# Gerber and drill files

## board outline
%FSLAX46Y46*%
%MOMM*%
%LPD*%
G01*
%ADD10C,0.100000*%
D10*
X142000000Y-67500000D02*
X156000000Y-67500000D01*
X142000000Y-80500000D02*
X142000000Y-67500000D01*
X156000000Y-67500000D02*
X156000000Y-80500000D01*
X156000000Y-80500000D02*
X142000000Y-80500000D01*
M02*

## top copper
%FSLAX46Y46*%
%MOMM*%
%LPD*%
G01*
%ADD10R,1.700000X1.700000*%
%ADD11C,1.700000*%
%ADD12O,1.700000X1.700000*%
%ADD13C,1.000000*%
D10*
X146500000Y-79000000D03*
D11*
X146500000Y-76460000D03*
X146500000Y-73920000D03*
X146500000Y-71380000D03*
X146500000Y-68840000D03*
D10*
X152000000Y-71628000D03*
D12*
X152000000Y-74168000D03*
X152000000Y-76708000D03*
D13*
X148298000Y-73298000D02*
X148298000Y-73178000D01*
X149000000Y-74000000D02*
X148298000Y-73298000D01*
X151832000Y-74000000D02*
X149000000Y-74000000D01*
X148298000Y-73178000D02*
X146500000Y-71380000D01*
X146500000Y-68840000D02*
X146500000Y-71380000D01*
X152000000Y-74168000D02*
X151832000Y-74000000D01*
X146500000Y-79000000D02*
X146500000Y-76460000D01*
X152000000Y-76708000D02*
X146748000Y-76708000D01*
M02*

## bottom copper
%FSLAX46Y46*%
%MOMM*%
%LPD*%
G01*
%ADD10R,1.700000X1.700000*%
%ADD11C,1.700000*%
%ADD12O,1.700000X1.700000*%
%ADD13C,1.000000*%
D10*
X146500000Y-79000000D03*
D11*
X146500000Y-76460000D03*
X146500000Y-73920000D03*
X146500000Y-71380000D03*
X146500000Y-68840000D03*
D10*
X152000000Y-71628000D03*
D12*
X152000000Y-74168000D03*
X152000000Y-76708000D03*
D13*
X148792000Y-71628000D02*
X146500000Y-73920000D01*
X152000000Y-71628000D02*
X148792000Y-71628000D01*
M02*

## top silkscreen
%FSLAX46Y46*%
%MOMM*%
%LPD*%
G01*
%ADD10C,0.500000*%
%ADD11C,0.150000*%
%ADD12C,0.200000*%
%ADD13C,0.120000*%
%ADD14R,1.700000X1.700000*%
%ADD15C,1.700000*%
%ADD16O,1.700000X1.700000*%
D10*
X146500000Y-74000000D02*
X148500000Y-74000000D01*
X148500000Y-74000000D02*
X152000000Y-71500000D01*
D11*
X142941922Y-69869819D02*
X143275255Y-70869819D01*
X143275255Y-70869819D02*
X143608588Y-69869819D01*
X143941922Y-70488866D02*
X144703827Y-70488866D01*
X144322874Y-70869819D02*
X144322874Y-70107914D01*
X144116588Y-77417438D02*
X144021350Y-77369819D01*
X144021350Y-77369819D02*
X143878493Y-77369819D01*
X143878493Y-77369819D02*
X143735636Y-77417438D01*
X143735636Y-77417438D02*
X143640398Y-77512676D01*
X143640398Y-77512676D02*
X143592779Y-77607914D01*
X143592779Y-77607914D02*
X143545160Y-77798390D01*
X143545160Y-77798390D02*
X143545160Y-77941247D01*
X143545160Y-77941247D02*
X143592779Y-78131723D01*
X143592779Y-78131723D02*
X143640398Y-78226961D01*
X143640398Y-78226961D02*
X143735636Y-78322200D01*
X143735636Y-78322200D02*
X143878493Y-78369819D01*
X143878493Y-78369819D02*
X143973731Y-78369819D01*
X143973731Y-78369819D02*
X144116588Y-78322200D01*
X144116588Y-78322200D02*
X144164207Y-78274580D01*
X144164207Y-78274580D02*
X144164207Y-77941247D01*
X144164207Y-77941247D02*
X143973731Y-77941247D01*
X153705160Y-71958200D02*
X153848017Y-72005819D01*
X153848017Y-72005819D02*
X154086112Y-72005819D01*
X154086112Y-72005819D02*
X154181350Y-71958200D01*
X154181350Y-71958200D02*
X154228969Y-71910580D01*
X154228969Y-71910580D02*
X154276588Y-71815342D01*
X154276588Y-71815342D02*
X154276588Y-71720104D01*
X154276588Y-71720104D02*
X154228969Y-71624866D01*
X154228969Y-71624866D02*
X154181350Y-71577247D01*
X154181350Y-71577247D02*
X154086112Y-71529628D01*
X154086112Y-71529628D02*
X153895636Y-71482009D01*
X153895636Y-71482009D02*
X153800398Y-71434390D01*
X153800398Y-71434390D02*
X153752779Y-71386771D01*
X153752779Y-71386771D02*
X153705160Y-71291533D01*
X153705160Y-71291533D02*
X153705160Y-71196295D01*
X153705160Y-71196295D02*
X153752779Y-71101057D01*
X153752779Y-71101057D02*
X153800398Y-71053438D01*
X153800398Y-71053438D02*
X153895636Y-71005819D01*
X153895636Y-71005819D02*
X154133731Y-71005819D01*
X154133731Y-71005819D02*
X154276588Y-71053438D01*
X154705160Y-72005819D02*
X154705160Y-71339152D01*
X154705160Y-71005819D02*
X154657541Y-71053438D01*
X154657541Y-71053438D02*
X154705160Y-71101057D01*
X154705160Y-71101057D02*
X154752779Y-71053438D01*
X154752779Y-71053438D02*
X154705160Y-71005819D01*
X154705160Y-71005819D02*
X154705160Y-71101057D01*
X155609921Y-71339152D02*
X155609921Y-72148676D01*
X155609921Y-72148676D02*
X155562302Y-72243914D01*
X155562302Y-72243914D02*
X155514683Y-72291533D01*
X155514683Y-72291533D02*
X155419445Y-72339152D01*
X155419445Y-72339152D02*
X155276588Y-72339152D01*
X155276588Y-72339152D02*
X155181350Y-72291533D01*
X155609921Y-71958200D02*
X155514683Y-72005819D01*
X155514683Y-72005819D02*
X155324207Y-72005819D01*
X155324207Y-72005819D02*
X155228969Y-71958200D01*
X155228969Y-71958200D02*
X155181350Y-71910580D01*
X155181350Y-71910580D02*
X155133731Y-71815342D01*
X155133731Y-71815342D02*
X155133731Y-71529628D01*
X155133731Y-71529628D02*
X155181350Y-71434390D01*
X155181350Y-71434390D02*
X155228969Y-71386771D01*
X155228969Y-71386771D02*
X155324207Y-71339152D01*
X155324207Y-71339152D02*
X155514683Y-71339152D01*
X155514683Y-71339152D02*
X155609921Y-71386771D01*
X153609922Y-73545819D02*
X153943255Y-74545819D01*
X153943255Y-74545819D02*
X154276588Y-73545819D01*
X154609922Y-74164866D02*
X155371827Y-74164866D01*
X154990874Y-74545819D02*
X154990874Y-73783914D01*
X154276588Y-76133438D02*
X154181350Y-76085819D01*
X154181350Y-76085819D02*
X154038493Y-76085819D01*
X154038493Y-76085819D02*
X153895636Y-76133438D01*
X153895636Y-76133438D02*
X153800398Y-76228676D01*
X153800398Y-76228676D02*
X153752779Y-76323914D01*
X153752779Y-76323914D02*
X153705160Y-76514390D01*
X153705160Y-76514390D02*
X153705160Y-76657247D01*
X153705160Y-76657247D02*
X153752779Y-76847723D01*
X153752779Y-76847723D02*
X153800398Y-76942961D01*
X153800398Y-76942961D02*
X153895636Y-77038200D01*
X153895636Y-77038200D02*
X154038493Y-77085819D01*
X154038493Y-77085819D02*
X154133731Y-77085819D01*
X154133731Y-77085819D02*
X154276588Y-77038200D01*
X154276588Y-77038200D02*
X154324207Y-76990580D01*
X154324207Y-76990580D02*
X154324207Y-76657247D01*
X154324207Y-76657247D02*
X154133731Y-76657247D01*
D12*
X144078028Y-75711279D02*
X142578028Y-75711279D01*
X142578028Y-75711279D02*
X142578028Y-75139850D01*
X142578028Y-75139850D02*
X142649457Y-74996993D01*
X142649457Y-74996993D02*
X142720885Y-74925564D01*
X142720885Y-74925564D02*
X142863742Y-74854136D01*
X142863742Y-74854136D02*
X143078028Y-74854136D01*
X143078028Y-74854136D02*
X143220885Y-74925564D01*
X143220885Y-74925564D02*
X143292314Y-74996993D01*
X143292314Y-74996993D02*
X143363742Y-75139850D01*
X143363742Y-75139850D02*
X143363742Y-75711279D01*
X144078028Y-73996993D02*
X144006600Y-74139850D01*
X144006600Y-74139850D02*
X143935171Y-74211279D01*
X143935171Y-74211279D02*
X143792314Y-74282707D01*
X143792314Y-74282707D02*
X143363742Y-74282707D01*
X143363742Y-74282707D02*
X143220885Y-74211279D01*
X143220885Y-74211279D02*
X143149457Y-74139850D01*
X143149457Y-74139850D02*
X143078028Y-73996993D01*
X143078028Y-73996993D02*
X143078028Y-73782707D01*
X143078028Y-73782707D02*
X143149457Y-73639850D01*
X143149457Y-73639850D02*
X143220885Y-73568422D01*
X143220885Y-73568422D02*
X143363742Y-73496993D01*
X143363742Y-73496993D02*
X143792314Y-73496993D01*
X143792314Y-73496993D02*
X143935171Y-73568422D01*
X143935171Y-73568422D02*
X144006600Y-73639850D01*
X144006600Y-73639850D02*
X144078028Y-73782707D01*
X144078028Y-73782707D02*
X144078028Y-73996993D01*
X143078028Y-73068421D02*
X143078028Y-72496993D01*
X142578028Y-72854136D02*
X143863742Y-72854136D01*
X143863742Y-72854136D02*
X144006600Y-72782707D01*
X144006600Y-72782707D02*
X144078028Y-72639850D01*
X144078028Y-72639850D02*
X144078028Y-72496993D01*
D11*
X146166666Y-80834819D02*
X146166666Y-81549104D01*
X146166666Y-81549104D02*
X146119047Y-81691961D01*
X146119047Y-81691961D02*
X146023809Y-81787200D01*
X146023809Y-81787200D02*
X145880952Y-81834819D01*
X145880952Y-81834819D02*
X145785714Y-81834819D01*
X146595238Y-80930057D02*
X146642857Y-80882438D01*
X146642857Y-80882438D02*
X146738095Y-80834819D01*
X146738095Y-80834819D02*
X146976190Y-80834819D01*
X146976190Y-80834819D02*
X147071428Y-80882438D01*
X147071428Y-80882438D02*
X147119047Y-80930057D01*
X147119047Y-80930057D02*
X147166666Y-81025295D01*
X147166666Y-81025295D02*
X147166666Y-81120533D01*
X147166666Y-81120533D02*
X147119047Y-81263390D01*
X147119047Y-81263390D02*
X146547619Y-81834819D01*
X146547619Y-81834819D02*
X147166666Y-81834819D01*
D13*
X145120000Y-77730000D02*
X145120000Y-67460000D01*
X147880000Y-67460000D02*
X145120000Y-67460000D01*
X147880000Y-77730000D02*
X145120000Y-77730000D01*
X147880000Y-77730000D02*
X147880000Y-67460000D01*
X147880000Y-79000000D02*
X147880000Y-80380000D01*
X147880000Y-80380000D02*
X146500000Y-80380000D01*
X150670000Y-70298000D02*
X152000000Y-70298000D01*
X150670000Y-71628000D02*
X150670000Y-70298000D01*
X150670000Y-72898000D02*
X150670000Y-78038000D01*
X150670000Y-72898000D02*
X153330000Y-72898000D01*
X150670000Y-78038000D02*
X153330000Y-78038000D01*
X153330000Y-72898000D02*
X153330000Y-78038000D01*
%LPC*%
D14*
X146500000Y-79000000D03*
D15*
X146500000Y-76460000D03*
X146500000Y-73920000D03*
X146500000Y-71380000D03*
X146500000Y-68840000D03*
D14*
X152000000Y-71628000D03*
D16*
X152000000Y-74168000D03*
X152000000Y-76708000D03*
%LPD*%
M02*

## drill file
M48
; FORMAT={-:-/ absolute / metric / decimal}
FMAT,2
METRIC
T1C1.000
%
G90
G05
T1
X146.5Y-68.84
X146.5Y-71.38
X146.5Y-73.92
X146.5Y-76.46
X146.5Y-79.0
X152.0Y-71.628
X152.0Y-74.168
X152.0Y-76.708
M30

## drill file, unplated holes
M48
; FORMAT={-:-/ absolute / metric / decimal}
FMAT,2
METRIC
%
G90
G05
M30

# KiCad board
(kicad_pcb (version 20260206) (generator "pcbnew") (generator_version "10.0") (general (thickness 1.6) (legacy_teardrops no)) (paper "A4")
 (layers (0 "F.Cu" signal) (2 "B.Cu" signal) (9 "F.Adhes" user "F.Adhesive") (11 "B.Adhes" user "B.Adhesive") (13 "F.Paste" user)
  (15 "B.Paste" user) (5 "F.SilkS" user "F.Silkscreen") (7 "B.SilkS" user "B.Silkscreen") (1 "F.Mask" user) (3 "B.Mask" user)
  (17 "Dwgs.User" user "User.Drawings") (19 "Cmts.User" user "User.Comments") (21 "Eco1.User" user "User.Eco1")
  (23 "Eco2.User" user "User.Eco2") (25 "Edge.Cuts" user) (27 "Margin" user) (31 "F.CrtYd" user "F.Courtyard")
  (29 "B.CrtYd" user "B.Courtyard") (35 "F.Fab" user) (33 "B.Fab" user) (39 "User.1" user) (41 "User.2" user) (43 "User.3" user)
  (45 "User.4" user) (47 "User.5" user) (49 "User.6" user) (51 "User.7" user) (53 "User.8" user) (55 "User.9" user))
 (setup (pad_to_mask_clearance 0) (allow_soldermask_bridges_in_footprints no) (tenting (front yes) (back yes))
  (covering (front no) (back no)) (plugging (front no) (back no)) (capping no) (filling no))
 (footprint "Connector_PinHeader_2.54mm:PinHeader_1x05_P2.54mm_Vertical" (layer "F.Cu") (at 146.5 79 180)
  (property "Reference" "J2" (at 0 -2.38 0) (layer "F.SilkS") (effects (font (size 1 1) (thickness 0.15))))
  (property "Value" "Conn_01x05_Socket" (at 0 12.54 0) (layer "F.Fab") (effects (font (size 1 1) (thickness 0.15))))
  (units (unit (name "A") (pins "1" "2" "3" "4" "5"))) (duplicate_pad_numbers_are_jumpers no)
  (fp_line (start 1.38 1.27) (end 1.38 11.54) (stroke (width 0.12) (type solid)) (layer "F.SilkS"))
  (fp_line (start -1.38 11.54) (end 1.38 11.54) (stroke (width 0.12) (type solid)) (layer "F.SilkS"))
  (fp_line (start -1.38 1.27) (end 1.38 1.27) (stroke (width 0.12) (type solid)) (layer "F.SilkS"))
  (fp_line (start -1.38 1.27) (end -1.38 11.54) (stroke (width 0.12) (type solid)) (layer "F.SilkS"))
  (fp_line (start -1.38 0) (end -1.38 -1.38) (stroke (width 0.12) (type solid)) (layer "F.SilkS"))
  (fp_line (start -1.38 -1.38) (end 0 -1.38) (stroke (width 0.12) (type solid)) (layer "F.SilkS"))
  (pad "1" thru_hole rect (at 0 0 180) (size 1.7 1.7) (drill 1) (layers "*.Cu" "*.Mask") (remove_unused_layers no) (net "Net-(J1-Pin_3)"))
  (pad "2" thru_hole circle (at 0 2.54 180) (size 1.7 1.7) (drill 1) (layers "*.Cu" "*.Mask") (remove_unused_layers no)
   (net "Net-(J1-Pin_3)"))
  (pad "3" thru_hole circle (at 0 5.08 180) (size 1.7 1.7) (drill 1) (layers "*.Cu" "*.Mask") (remove_unused_layers no)
   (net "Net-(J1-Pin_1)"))
  (pad "4" thru_hole circle (at 0 7.62 180) (size 1.7 1.7) (drill 1) (layers "*.Cu" "*.Mask") (remove_unused_layers no)
   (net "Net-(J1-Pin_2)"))
  (pad "5" thru_hole circle (at 0 10.16 180) (size 1.7 1.7) (drill 1) (layers "*.Cu" "*.Mask") (remove_unused_layers no)
   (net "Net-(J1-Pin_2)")))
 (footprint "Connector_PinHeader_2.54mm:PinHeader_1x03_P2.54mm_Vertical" (layer "F.Cu") (at 152 71.628)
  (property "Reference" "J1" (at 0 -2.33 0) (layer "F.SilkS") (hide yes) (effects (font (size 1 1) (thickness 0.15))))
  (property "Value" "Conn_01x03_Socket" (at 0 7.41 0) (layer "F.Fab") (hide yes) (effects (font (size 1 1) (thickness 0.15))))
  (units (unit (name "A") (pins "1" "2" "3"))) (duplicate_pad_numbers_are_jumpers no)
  (fp_line (start -1.33 -1.33) (end 0 -1.33) (stroke (width 0.12) (type solid)) (layer "F.SilkS"))
  (fp_line (start -1.33 0) (end -1.33 -1.33) (stroke (width 0.12) (type solid)) (layer "F.SilkS"))
  (fp_line (start -1.33 1.27) (end -1.33 6.41) (stroke (width 0.12) (type solid)) (layer "F.SilkS"))
  (fp_line (start -1.33 1.27) (end 1.33 1.27) (stroke (width 0.12) (type solid)) (layer "F.SilkS"))
  (fp_line (start -1.33 6.41) (end 1.33 6.41) (stroke (width 0.12) (type solid)) (layer "F.SilkS"))
  (fp_line (start 1.33 1.27) (end 1.33 6.41) (stroke (width 0.12) (type solid)) (layer "F.SilkS"))
  (pad "1" thru_hole rect (at 0 0) (size 1.7 1.7) (drill 1) (layers "*.Cu" "*.Mask") (remove_unused_layers no) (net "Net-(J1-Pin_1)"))
  (pad "2" thru_hole oval (at 0 2.54) (size 1.7 1.7) (drill 1) (layers "*.Cu" "*.Mask") (remove_unused_layers no) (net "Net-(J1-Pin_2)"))
  (pad "3" thru_hole oval (at 0 5.08) (size 1.7 1.7) (drill 1) (layers "*.Cu" "*.Mask") (remove_unused_layers no) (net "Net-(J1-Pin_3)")))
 (gr_line (start 146.5 74) (end 148.5 74) (stroke (width 0.5) (type solid)) (layer "F.SilkS"))
 (gr_line (start 148.5 74) (end 152 71.5) (stroke (width 0.5) (type solid)) (layer "F.SilkS"))
 (gr_line (start 142 67.5) (end 156 67.5) (stroke (width 0.1) (type solid)) (layer "Edge.Cuts"))
 (gr_line (start 142 80.5) (end 142 67.5) (stroke (width 0.1) (type solid)) (layer "Edge.Cuts"))
 (gr_line (start 156 67.5) (end 156 80.5) (stroke (width 0.1) (type solid)) (layer "Edge.Cuts"))
 (gr_line (start 156 80.5) (end 142 80.5) (stroke (width 0.1) (type solid)) (layer "Edge.Cuts"))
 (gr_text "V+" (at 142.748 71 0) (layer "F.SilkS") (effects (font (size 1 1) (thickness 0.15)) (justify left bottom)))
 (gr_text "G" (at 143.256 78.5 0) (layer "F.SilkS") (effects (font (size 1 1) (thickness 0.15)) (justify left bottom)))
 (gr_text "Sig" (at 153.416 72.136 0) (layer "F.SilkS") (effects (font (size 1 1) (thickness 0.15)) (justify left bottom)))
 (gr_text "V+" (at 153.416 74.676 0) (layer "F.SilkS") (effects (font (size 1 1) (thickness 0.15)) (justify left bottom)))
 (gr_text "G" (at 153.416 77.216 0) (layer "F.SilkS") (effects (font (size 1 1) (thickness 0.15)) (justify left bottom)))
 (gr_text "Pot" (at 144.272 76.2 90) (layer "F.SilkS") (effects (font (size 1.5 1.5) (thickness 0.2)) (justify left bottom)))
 (segment (start 146.5 79) (end 146.5 76.46) (width 1) (layer "F.Cu") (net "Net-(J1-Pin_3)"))
 (segment (start 152 76.708) (end 146.748 76.708) (width 1) (layer "F.Cu") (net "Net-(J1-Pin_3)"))
 (segment (start 148.792 71.628) (end 146.5 73.92) (width 1) (layer "B.Cu") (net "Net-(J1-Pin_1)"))
 (segment (start 152 71.628) (end 148.792 71.628) (width 1) (layer "B.Cu") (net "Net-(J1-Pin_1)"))
 (segment (start 148.298 73.298) (end 148.298 73.178) (width 1) (layer "F.Cu") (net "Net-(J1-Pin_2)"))
 (segment (start 149 74) (end 148.298 73.298) (width 1) (layer "F.Cu") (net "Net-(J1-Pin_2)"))
 (segment (start 151.832 74) (end 149 74) (width 1) (layer "F.Cu") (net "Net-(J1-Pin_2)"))
 (segment (start 148.298 73.178) (end 146.5 71.38) (width 1) (layer "F.Cu") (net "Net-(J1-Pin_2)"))
 (segment (start 146.5 68.84) (end 146.5 71.38) (width 1) (layer "F.Cu") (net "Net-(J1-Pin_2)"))
 (segment (start 152 74.168) (end 151.832 74) (width 1) (layer "F.Cu") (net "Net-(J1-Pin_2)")))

